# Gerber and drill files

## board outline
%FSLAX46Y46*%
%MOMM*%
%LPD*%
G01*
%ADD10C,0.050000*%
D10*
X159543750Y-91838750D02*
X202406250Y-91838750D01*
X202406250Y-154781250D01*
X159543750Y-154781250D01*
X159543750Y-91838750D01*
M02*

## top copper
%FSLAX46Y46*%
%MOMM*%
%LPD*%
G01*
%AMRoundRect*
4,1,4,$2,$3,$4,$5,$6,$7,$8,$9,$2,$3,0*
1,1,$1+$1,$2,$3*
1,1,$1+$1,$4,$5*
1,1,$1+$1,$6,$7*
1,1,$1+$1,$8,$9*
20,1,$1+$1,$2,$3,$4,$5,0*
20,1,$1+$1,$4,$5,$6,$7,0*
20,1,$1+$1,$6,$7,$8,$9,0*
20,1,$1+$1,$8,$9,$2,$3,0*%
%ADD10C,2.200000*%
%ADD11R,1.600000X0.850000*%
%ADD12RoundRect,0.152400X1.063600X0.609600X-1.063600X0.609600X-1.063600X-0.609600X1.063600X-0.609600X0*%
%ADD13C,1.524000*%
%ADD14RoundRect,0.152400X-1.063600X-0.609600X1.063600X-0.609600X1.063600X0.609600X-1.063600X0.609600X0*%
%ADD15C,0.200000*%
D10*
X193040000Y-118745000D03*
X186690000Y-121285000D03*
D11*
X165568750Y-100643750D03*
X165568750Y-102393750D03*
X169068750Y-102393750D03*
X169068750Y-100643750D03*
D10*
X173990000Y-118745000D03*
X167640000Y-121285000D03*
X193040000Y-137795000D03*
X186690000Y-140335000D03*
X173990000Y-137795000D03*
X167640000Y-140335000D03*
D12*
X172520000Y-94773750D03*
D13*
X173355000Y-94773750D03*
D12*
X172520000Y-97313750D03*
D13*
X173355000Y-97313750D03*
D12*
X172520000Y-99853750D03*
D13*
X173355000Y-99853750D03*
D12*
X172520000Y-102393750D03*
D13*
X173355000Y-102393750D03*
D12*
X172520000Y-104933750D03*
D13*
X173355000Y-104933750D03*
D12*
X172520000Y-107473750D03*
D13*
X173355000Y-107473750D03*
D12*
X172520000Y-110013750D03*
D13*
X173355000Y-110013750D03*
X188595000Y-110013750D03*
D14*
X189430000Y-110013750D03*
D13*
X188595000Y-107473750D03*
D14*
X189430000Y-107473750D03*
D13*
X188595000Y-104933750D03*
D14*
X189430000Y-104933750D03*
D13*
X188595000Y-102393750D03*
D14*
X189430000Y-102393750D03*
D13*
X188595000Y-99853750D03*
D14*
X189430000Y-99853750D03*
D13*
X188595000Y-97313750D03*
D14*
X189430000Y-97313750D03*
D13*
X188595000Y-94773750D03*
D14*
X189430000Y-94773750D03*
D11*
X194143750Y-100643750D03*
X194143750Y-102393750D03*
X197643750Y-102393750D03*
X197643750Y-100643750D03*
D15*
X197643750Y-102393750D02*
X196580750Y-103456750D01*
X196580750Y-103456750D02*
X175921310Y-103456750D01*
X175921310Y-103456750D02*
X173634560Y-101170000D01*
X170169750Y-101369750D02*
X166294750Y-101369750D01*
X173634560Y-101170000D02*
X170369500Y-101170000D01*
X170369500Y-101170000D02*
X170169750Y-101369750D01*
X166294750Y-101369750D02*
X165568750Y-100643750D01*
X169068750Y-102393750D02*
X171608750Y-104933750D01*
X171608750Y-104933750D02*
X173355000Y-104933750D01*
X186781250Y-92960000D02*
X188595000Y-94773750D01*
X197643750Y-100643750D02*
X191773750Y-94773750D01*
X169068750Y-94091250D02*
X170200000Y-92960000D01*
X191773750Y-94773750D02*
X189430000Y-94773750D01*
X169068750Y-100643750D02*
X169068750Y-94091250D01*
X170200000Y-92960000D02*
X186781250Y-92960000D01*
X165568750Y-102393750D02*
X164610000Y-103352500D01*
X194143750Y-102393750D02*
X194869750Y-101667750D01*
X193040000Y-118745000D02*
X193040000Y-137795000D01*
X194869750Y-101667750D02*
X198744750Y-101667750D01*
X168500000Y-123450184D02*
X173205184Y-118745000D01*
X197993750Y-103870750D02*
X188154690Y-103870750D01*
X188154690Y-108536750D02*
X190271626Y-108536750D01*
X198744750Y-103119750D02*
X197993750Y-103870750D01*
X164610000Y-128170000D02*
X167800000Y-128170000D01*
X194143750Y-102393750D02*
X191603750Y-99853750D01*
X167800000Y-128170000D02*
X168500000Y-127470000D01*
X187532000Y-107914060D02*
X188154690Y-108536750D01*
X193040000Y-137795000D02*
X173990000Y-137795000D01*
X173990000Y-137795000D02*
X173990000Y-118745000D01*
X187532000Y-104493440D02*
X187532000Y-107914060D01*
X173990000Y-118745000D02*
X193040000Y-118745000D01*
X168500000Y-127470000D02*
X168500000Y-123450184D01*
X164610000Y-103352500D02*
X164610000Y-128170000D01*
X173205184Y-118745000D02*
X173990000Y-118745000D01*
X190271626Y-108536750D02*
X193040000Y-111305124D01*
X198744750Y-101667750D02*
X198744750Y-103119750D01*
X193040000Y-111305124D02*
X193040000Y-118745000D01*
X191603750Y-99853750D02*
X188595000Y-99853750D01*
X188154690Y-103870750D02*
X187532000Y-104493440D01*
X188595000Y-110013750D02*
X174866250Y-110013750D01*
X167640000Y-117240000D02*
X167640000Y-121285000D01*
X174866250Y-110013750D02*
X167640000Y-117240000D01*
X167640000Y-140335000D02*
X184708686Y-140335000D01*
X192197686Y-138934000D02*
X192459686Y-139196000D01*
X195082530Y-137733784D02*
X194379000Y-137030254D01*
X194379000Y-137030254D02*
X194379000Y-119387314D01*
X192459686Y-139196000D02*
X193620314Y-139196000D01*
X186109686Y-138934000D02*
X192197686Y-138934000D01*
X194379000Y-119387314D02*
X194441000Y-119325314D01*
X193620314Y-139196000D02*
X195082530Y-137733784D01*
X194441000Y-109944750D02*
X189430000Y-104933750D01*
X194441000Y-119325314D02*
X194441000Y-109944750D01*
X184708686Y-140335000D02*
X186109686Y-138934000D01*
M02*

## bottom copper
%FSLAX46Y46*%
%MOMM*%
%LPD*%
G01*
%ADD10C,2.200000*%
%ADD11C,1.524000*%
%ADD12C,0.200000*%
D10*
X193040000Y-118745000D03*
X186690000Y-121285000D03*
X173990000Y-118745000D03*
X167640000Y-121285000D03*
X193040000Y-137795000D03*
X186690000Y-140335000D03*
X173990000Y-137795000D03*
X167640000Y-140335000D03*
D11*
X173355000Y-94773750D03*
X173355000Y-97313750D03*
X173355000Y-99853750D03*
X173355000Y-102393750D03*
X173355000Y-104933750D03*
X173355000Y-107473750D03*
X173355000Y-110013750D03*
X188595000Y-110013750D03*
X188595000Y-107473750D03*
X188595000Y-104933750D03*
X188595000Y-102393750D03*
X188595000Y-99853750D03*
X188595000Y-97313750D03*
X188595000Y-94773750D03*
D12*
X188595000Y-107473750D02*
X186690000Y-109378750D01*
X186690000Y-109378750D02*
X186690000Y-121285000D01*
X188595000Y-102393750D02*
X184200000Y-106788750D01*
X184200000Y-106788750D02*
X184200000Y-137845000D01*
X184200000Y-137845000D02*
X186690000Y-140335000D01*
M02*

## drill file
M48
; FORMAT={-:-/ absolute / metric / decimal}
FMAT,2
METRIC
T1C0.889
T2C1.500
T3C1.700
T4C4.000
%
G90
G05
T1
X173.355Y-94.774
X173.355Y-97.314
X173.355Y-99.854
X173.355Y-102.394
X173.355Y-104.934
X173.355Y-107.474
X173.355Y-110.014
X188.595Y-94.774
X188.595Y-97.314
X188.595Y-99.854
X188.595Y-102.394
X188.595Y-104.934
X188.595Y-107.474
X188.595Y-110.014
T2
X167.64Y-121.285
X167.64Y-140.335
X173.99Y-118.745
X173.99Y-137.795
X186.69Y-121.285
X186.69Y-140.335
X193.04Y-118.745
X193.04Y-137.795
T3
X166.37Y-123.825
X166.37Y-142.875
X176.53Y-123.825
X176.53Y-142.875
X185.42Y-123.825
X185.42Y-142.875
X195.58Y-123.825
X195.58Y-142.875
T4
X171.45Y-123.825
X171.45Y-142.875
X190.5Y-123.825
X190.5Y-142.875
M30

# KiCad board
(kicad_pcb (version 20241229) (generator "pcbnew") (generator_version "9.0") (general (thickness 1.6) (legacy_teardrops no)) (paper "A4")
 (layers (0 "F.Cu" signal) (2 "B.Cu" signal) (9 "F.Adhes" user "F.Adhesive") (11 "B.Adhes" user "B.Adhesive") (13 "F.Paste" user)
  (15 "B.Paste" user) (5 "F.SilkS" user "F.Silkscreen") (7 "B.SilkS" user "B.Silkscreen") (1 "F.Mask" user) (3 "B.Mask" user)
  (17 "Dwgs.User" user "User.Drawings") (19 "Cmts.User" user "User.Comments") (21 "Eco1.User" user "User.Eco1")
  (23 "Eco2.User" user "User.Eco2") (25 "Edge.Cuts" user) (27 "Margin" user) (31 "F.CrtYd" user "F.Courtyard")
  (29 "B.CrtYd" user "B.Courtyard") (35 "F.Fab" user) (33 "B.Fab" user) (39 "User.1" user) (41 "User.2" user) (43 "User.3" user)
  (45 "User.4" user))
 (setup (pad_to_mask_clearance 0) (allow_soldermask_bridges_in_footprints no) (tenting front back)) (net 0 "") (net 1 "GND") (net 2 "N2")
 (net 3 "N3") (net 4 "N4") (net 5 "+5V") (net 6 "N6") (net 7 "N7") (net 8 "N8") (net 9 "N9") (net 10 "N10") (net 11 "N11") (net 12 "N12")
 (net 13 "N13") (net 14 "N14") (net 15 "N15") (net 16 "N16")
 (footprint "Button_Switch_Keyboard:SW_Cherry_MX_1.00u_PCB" (layer "F.Cu") (at 193.04 118.745)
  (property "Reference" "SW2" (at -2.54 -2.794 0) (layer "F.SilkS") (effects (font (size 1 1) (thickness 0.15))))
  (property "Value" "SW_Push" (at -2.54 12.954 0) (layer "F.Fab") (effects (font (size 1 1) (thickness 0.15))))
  (pad "" np_thru_hole circle (at -7.62 5.08) (size 1.7 1.7) (drill 1.7) (layers "*.Cu" "*.Mask"))
  (pad "" np_thru_hole circle (at -2.54 5.08) (size 4 4) (drill 4) (layers "*.Cu" "*.Mask"))
  (pad "" np_thru_hole circle (at 2.54 5.08) (size 1.7 1.7) (drill 1.7) (layers "*.Cu" "*.Mask"))
  (pad "1" thru_hole circle (at 0 0) (size 2.2 2.2) (drill 1.5) (layers "*.Cu" "*.Mask") (remove_unused_layers no) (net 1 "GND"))
  (pad "2" thru_hole circle (at -6.35 2.54) (size 2.2 2.2) (drill 1.5) (layers "*.Cu" "*.Mask") (remove_unused_layers no) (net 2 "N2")))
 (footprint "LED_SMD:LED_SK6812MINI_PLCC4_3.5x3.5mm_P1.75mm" (layer "F.Cu") (at 167.31875 101.51875)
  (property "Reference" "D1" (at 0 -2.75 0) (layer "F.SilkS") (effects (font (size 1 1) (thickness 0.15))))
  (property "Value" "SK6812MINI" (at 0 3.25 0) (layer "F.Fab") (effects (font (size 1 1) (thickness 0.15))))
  (pad "1" smd rect (at -1.75 -0.875) (size 1.6 0.85) (layers "F.Cu" "F.Mask" "F.Paste") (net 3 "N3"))
  (pad "2" smd rect (at -1.75 0.875) (size 1.6 0.85) (layers "F.Cu" "F.Mask" "F.Paste") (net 1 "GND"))
  (pad "3" smd rect (at 1.75 0.875) (size 1.6 0.85) (layers "F.Cu" "F.Mask" "F.Paste") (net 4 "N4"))
  (pad "4" smd rect (at 1.75 -0.875) (size 1.6 0.85) (layers "F.Cu" "F.Mask" "F.Paste") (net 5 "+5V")))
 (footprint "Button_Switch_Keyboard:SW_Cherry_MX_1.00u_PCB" (layer "F.Cu") (at 173.99 118.745)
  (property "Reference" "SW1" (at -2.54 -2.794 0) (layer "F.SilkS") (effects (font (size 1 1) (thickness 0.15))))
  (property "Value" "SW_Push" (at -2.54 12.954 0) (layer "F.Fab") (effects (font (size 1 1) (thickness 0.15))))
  (pad "" np_thru_hole circle (at -7.62 5.08) (size 1.7 1.7) (drill 1.7) (layers "*.Cu" "*.Mask"))
  (pad "" np_thru_hole circle (at -2.54 5.08) (size 4 4) (drill 4) (layers "*.Cu" "*.Mask"))
  (pad "" np_thru_hole circle (at 2.54 5.08) (size 1.7 1.7) (drill 1.7) (layers "*.Cu" "*.Mask"))
  (pad "1" thru_hole circle (at 0 0) (size 2.2 2.2) (drill 1.5) (layers "*.Cu" "*.Mask") (remove_unused_layers no) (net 1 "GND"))
  (pad "2" thru_hole circle (at -6.35 2.54) (size 2.2 2.2) (drill 1.5) (layers "*.Cu" "*.Mask") (remove_unused_layers no) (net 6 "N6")))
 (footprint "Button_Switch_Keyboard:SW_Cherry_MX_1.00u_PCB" (layer "F.Cu") (at 193.04 137.795)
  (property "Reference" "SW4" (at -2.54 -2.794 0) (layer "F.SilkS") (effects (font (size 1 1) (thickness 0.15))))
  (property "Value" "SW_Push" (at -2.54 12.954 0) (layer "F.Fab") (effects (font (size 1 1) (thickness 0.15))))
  (pad "" np_thru_hole circle (at -7.62 5.08) (size 1.7 1.7) (drill 1.7) (layers "*.Cu" "*.Mask"))
  (pad "" np_thru_hole circle (at -2.54 5.08) (size 4 4) (drill 4) (layers "*.Cu" "*.Mask"))
  (pad "" np_thru_hole circle (at 2.54 5.08) (size 1.7 1.7) (drill 1.7) (layers "*.Cu" "*.Mask"))
  (pad "1" thru_hole circle (at 0 0) (size 2.2 2.2) (drill 1.5) (layers "*.Cu" "*.Mask") (remove_unused_layers no) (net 1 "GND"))
  (pad "2" thru_hole circle (at -6.35 2.54) (size 2.2 2.2) (drill 1.5) (layers "*.Cu" "*.Mask") (remove_unused_layers no) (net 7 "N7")))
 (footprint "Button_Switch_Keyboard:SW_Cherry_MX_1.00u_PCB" (layer "F.Cu") (at 173.99 137.795)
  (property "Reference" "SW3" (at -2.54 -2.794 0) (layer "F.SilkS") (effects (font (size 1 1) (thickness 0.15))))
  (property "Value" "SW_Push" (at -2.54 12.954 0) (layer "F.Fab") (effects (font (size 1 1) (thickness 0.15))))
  (pad "" np_thru_hole circle (at -7.62 5.08) (size 1.7 1.7) (drill 1.7) (layers "*.Cu" "*.Mask"))
  (pad "" np_thru_hole circle (at -2.54 5.08) (size 4 4) (drill 4) (layers "*.Cu" "*.Mask"))
  (pad "" np_thru_hole circle (at 2.54 5.08) (size 1.7 1.7) (drill 1.7) (layers "*.Cu" "*.Mask"))
  (pad "1" thru_hole circle (at 0 0) (size 2.2 2.2) (drill 1.5) (layers "*.Cu" "*.Mask") (remove_unused_layers no) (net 1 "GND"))
  (pad "2" thru_hole circle (at -6.35 2.54) (size 2.2 2.2) (drill 1.5) (layers "*.Cu" "*.Mask") (remove_unused_layers no) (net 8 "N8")))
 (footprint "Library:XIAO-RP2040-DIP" (layer "F.Cu") (at 180.975 102.39375)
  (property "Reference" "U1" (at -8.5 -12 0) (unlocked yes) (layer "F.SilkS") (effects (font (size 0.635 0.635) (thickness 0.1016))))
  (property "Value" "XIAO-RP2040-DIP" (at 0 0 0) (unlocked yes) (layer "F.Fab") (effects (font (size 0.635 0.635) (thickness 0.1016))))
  (pad "1" smd roundrect (at -8.455 -7.62 180) (size 2.432 1.524) (layers "F.Cu" "F.Mask") (roundrect_rratio 0.1) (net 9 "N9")
   (thermal_bridge_angle 45))
  (pad "1" thru_hole circle (at -7.62 -7.62 180) (size 1.524 1.524) (drill 0.889) (layers "*.Cu" "*.Mask") (remove_unused_layers no)
   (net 9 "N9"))
  (pad "2" smd roundrect (at -8.455 -5.08 180) (size 2.432 1.524) (layers "F.Cu" "F.Mask") (roundrect_rratio 0.1) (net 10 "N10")
   (thermal_bridge_angle 45))
  (pad "2" thru_hole circle (at -7.62 -5.08 180) (size 1.524 1.524) (drill 0.889) (layers "*.Cu" "*.Mask") (remove_unused_layers no)
   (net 10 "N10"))
  (pad "3" smd roundrect (at -8.455 -2.54 180) (size 2.432 1.524) (layers "F.Cu" "F.Mask") (roundrect_rratio 0.1) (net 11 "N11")
   (thermal_bridge_angle 45))
  (pad "3" thru_hole circle (at -7.62 -2.54 180) (size 1.524 1.524) (drill 0.889) (layers "*.Cu" "*.Mask") (remove_unused_layers no)
   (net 11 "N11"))
  (pad "4" smd roundrect (at -8.455 0 180) (size 2.432 1.524) (layers "F.Cu" "F.Mask") (roundrect_rratio 0.1) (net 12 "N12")
   (thermal_bridge_angle 45))
  (pad "4" thru_hole circle (at -7.62 0 180) (size 1.524 1.524) (drill 0.889) (layers "*.Cu" "*.Mask") (remove_unused_layers no)
   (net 12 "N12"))
  (pad "5" smd roundrect (at -8.455 2.54 180) (size 2.432 1.524) (layers "F.Cu" "F.Mask") (roundrect_rratio 0.1) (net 4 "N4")
   (thermal_bridge_angle 45))
  (pad "5" thru_hole circle (at -7.62 2.54 180) (size 1.524 1.524) (drill 0.889) (layers "*.Cu" "*.Mask") (remove_unused_layers no)
   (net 4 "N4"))
  (pad "6" smd roundrect (at -8.455 5.08 180) (size 2.432 1.524) (layers "F.Cu" "F.Mask") (roundrect_rratio 0.1) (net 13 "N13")
   (thermal_bridge_angle 45))
  (pad "6" thru_hole circle (at -7.62 5.08 180) (size 1.524 1.524) (drill 0.889) (layers "*.Cu" "*.Mask") (remove_unused_layers no)
   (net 13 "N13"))
  (pad "7" smd roundrect (at -8.455 7.62 180) (size 2.432 1.524) (layers "F.Cu" "F.Mask") (roundrect_rratio 0.1) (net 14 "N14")
   (thermal_bridge_angle 45))
  (pad "7" thru_hole circle (at -7.62 7.62 180) (size 1.524 1.524) (drill 0.889) (layers "*.Cu" "*.Mask") (remove_unused_layers no)
   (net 14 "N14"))
  (pad "8" thru_hole circle (at 7.62 7.62) (size 1.524 1.524) (drill 0.889) (layers "*.Cu" "*.Mask") (remove_unused_layers no) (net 6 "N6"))
  (pad "8" smd roundrect (at 8.455 7.62) (size 2.432 1.524) (layers "F.Cu" "F.Mask") (roundrect_rratio 0.1) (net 6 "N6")
   (thermal_bridge_angle 45))
  (pad "9" thru_hole circle (at 7.62 5.08) (size 1.524 1.524) (drill 0.889) (layers "*.Cu" "*.Mask") (remove_unused_layers no) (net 2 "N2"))
  (pad "9" smd roundrect (at 8.455 5.08) (size 2.432 1.524) (layers "F.Cu" "F.Mask") (roundrect_rratio 0.1) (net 2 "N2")
   (thermal_bridge_angle 45))
  (pad "10" thru_hole circle (at 7.62 2.54) (size 1.524 1.524) (drill 0.889) (layers "*.Cu" "*.Mask") (remove_unused_layers no) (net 8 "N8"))
  (pad "10" smd roundrect (at 8.455 2.54) (size 2.432 1.524) (layers "F.Cu" "F.Mask") (roundrect_rratio 0.1) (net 8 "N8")
   (thermal_bridge_angle 45))
  (pad "11" thru_hole circle (at 7.62 0) (size 1.524 1.524) (drill 0.889) (layers "*.Cu" "*.Mask") (remove_unused_layers no) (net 7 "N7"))
  (pad "11" smd roundrect (at 8.455 0) (size 2.432 1.524) (layers "F.Cu" "F.Mask") (roundrect_rratio 0.1) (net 7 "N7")
   (thermal_bridge_angle 45))
  (pad "12" thru_hole circle (at 7.62 -2.54) (size 1.524 1.524) (drill 0.889) (layers "*.Cu" "*.Mask") (remove_unused_layers no)
   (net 1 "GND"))
  (pad "12" smd roundrect (at 8.455 -2.54) (size 2.432 1.524) (layers "F.Cu" "F.Mask") (roundrect_rratio 0.1) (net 1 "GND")
   (thermal_bridge_angle 45))
  (pad "13" thru_hole circle (at 7.62 -5.08) (size 1.524 1.524) (drill 0.889) (layers "*.Cu" "*.Mask") (remove_unused_layers no)
   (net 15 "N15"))
  (pad "13" smd roundrect (at 8.455 -5.08) (size 2.432 1.524) (layers "F.Cu" "F.Mask") (roundrect_rratio 0.1) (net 15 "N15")
   (thermal_bridge_angle 45))
  (pad "14" thru_hole circle (at 7.62 -7.62) (size 1.524 1.524) (drill 0.889) (layers "*.Cu" "*.Mask") (remove_unused_layers no)
   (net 5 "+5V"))
  (pad "14" smd roundrect (at 8.455 -7.62) (size 2.432 1.524) (layers "F.Cu" "F.Mask") (roundrect_rratio 0.1) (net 5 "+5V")
   (thermal_bridge_angle 45)))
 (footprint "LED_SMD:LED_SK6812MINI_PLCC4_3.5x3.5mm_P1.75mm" (layer "F.Cu") (at 195.89375 101.51875)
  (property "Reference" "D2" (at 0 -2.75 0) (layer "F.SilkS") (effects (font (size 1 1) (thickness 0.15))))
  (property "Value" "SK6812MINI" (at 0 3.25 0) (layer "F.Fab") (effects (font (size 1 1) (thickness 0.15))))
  (pad "1" smd rect (at -1.75 -0.875) (size 1.6 0.85) (layers "F.Cu" "F.Mask" "F.Paste") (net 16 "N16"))
  (pad "2" smd rect (at -1.75 0.875) (size 1.6 0.85) (layers "F.Cu" "F.Mask" "F.Paste") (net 1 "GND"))
  (pad "3" smd rect (at 1.75 0.875) (size 1.6 0.85) (layers "F.Cu" "F.Mask" "F.Paste") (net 3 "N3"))
  (pad "4" smd rect (at 1.75 -0.875) (size 1.6 0.85) (layers "F.Cu" "F.Mask" "F.Paste") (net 5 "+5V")))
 (gr_rect (start 159.54375 91.83875) (end 202.40625 154.78125) (stroke (width 0.05) (type default)) (fill no) (layer "Edge.Cuts"))
 (segment (start 197.64375 102.39375) (end 196.58075 103.45675) (width 0.2) (layer "F.Cu") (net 3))
 (segment (start 196.58075 103.45675) (end 175.92131 103.45675) (width 0.2) (layer "F.Cu") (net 3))
 (segment (start 175.92131 103.45675) (end 173.63456 101.17) (width 0.2) (layer "F.Cu") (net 3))
 (segment (start 170.16975 101.36975) (end 166.29475 101.36975) (width 0.2) (layer "F.Cu") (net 3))
 (segment (start 173.63456 101.17) (end 170.3695 101.17) (width 0.2) (layer "F.Cu") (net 3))
 (segment (start 170.3695 101.17) (end 170.16975 101.36975) (width 0.2) (layer "F.Cu") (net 3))
 (segment (start 166.29475 101.36975) (end 165.56875 100.64375) (width 0.2) (layer "F.Cu") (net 3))
 (segment (start 169.06875 102.39375) (end 171.60875 104.93375) (width 0.2) (layer "F.Cu") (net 4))
 (segment (start 171.60875 104.93375) (end 173.355 104.93375) (width 0.2) (layer "F.Cu") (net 4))
 (segment (start 186.78125 92.96) (end 188.595 94.77375) (width 0.2) (layer "F.Cu") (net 5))
 (segment (start 197.64375 100.64375) (end 191.77375 94.77375) (width 0.2) (layer "F.Cu") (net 5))
 (segment (start 169.06875 94.09125) (end 170.2 92.96) (width 0.2) (layer "F.Cu") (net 5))
 (segment (start 191.77375 94.77375) (end 189.43 94.77375) (width 0.2) (layer "F.Cu") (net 5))
 (segment (start 169.06875 100.64375) (end 169.06875 94.09125) (width 0.2) (layer "F.Cu") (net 5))
 (segment (start 170.2 92.96) (end 186.78125 92.96) (width 0.2) (layer "F.Cu") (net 5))
 (segment (start 165.56875 102.39375) (end 164.61 103.3525) (width 0.2) (layer "F.Cu") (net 1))
 (segment (start 194.14375 102.39375) (end 194.86975 101.66775) (width 0.2) (layer "F.Cu") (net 1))
 (segment (start 193.04 118.745) (end 193.04 137.795) (width 0.2) (layer "F.Cu") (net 1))
 (segment (start 194.86975 101.66775) (end 198.74475 101.66775) (width 0.2) (layer "F.Cu") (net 1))
 (segment (start 168.5 123.450184) (end 173.205184 118.745) (width 0.2) (layer "F.Cu") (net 1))
 (segment (start 197.99375 103.87075) (end 188.15469 103.87075) (width 0.2) (layer "F.Cu") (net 1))
 (segment (start 188.15469 108.53675) (end 190.271626 108.53675) (width 0.2) (layer "F.Cu") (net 1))
 (segment (start 198.74475 103.11975) (end 197.99375 103.87075) (width 0.2) (layer "F.Cu") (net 1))
 (segment (start 164.61 128.17) (end 167.8 128.17) (width 0.2) (layer "F.Cu") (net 1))
 (segment (start 194.14375 102.39375) (end 191.60375 99.85375) (width 0.2) (layer "F.Cu") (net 1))
 (segment (start 167.8 128.17) (end 168.5 127.47) (width 0.2) (layer "F.Cu") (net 1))
 (segment (start 187.532 107.91406) (end 188.15469 108.53675) (width 0.2) (layer "F.Cu") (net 1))
 (segment (start 193.04 137.795) (end 173.99 137.795) (width 0.2) (layer "F.Cu") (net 1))
 (segment (start 173.99 137.795) (end 173.99 118.745) (width 0.2) (layer "F.Cu") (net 1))
 (segment (start 187.532 104.49344) (end 187.532 107.91406) (width 0.2) (layer "F.Cu") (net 1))
 (segment (start 173.99 118.745) (end 193.04 118.745) (width 0.2) (layer "F.Cu") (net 1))
 (segment (start 168.5 127.47) (end 168.5 123.450184) (width 0.2) (layer "F.Cu") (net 1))
 (segment (start 164.61 103.3525) (end 164.61 128.17) (width 0.2) (layer "F.Cu") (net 1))
 (segment (start 173.205184 118.745) (end 173.99 118.745) (width 0.2) (layer "F.Cu") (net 1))
 (segment (start 190.271626 108.53675) (end 193.04 111.305124) (width 0.2) (layer "F.Cu") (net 1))
 (segment (start 198.74475 101.66775) (end 198.74475 103.11975) (width 0.2) (layer "F.Cu") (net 1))
 (segment (start 193.04 111.305124) (end 193.04 118.745) (width 0.2) (layer "F.Cu") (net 1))
 (segment (start 191.60375 99.85375) (end 188.595 99.85375) (width 0.2) (layer "F.Cu") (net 1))
 (segment (start 188.15469 103.87075) (end 187.532 104.49344) (width 0.2) (layer "F.Cu") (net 1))
 (segment (start 188.595 110.01375) (end 174.86625 110.01375) (width 0.2) (layer "F.Cu") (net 6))
 (segment (start 167.64 117.24) (end 167.64 121.285) (width 0.2) (layer "F.Cu") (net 6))
 (segment (start 174.86625 110.01375) (end 167.64 117.24) (width 0.2) (layer "F.Cu") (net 6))
 (segment (start 188.595 107.47375) (end 186.69 109.37875) (width 0.2) (layer "B.Cu") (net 2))
 (segment (start 186.69 109.37875) (end 186.69 121.285) (width 0.2) (layer "B.Cu") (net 2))
 (segment (start 167.64 140.335) (end 184.708686 140.335) (width 0.2) (layer "F.Cu") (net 8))
 (segment (start 192.197686 138.934) (end 192.459686 139.196) (width 0.2) (layer "F.Cu") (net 8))
 (segment (start 195.08253 137.733784) (end 194.379 137.030254) (width 0.2) (layer "F.Cu") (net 8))
 (segment (start 194.379 137.030254) (end 194.379 119.387314) (width 0.2) (layer "F.Cu") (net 8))
 (segment (start 192.459686 139.196) (end 193.620314 139.196) (width 0.2) (layer "F.Cu") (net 8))
 (segment (start 186.109686 138.934) (end 192.197686 138.934) (width 0.2) (layer "F.Cu") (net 8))
 (segment (start 194.379 119.387314) (end 194.441 119.325314) (width 0.2) (layer "F.Cu") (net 8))
 (segment (start 193.620314 139.196) (end 195.08253 137.733784) (width 0.2) (layer "F.Cu") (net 8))
 (segment (start 194.441 109.94475) (end 189.43 104.93375) (width 0.2) (layer "F.Cu") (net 8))
 (segment (start 194.441 119.325314) (end 194.441 109.94475) (width 0.2) (layer "F.Cu") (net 8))
 (segment (start 184.708686 140.335) (end 186.109686 138.934) (width 0.2) (layer "F.Cu") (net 8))
 (segment (start 188.595 102.39375) (end 184.2 106.78875) (width 0.2) (layer "B.Cu") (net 7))
 (segment (start 184.2 106.78875) (end 184.2 137.845) (width 0.2) (layer "B.Cu") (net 7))
 (segment (start 184.2 137.845) (end 186.69 140.335) (width 0.2) (layer "B.Cu") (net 7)))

